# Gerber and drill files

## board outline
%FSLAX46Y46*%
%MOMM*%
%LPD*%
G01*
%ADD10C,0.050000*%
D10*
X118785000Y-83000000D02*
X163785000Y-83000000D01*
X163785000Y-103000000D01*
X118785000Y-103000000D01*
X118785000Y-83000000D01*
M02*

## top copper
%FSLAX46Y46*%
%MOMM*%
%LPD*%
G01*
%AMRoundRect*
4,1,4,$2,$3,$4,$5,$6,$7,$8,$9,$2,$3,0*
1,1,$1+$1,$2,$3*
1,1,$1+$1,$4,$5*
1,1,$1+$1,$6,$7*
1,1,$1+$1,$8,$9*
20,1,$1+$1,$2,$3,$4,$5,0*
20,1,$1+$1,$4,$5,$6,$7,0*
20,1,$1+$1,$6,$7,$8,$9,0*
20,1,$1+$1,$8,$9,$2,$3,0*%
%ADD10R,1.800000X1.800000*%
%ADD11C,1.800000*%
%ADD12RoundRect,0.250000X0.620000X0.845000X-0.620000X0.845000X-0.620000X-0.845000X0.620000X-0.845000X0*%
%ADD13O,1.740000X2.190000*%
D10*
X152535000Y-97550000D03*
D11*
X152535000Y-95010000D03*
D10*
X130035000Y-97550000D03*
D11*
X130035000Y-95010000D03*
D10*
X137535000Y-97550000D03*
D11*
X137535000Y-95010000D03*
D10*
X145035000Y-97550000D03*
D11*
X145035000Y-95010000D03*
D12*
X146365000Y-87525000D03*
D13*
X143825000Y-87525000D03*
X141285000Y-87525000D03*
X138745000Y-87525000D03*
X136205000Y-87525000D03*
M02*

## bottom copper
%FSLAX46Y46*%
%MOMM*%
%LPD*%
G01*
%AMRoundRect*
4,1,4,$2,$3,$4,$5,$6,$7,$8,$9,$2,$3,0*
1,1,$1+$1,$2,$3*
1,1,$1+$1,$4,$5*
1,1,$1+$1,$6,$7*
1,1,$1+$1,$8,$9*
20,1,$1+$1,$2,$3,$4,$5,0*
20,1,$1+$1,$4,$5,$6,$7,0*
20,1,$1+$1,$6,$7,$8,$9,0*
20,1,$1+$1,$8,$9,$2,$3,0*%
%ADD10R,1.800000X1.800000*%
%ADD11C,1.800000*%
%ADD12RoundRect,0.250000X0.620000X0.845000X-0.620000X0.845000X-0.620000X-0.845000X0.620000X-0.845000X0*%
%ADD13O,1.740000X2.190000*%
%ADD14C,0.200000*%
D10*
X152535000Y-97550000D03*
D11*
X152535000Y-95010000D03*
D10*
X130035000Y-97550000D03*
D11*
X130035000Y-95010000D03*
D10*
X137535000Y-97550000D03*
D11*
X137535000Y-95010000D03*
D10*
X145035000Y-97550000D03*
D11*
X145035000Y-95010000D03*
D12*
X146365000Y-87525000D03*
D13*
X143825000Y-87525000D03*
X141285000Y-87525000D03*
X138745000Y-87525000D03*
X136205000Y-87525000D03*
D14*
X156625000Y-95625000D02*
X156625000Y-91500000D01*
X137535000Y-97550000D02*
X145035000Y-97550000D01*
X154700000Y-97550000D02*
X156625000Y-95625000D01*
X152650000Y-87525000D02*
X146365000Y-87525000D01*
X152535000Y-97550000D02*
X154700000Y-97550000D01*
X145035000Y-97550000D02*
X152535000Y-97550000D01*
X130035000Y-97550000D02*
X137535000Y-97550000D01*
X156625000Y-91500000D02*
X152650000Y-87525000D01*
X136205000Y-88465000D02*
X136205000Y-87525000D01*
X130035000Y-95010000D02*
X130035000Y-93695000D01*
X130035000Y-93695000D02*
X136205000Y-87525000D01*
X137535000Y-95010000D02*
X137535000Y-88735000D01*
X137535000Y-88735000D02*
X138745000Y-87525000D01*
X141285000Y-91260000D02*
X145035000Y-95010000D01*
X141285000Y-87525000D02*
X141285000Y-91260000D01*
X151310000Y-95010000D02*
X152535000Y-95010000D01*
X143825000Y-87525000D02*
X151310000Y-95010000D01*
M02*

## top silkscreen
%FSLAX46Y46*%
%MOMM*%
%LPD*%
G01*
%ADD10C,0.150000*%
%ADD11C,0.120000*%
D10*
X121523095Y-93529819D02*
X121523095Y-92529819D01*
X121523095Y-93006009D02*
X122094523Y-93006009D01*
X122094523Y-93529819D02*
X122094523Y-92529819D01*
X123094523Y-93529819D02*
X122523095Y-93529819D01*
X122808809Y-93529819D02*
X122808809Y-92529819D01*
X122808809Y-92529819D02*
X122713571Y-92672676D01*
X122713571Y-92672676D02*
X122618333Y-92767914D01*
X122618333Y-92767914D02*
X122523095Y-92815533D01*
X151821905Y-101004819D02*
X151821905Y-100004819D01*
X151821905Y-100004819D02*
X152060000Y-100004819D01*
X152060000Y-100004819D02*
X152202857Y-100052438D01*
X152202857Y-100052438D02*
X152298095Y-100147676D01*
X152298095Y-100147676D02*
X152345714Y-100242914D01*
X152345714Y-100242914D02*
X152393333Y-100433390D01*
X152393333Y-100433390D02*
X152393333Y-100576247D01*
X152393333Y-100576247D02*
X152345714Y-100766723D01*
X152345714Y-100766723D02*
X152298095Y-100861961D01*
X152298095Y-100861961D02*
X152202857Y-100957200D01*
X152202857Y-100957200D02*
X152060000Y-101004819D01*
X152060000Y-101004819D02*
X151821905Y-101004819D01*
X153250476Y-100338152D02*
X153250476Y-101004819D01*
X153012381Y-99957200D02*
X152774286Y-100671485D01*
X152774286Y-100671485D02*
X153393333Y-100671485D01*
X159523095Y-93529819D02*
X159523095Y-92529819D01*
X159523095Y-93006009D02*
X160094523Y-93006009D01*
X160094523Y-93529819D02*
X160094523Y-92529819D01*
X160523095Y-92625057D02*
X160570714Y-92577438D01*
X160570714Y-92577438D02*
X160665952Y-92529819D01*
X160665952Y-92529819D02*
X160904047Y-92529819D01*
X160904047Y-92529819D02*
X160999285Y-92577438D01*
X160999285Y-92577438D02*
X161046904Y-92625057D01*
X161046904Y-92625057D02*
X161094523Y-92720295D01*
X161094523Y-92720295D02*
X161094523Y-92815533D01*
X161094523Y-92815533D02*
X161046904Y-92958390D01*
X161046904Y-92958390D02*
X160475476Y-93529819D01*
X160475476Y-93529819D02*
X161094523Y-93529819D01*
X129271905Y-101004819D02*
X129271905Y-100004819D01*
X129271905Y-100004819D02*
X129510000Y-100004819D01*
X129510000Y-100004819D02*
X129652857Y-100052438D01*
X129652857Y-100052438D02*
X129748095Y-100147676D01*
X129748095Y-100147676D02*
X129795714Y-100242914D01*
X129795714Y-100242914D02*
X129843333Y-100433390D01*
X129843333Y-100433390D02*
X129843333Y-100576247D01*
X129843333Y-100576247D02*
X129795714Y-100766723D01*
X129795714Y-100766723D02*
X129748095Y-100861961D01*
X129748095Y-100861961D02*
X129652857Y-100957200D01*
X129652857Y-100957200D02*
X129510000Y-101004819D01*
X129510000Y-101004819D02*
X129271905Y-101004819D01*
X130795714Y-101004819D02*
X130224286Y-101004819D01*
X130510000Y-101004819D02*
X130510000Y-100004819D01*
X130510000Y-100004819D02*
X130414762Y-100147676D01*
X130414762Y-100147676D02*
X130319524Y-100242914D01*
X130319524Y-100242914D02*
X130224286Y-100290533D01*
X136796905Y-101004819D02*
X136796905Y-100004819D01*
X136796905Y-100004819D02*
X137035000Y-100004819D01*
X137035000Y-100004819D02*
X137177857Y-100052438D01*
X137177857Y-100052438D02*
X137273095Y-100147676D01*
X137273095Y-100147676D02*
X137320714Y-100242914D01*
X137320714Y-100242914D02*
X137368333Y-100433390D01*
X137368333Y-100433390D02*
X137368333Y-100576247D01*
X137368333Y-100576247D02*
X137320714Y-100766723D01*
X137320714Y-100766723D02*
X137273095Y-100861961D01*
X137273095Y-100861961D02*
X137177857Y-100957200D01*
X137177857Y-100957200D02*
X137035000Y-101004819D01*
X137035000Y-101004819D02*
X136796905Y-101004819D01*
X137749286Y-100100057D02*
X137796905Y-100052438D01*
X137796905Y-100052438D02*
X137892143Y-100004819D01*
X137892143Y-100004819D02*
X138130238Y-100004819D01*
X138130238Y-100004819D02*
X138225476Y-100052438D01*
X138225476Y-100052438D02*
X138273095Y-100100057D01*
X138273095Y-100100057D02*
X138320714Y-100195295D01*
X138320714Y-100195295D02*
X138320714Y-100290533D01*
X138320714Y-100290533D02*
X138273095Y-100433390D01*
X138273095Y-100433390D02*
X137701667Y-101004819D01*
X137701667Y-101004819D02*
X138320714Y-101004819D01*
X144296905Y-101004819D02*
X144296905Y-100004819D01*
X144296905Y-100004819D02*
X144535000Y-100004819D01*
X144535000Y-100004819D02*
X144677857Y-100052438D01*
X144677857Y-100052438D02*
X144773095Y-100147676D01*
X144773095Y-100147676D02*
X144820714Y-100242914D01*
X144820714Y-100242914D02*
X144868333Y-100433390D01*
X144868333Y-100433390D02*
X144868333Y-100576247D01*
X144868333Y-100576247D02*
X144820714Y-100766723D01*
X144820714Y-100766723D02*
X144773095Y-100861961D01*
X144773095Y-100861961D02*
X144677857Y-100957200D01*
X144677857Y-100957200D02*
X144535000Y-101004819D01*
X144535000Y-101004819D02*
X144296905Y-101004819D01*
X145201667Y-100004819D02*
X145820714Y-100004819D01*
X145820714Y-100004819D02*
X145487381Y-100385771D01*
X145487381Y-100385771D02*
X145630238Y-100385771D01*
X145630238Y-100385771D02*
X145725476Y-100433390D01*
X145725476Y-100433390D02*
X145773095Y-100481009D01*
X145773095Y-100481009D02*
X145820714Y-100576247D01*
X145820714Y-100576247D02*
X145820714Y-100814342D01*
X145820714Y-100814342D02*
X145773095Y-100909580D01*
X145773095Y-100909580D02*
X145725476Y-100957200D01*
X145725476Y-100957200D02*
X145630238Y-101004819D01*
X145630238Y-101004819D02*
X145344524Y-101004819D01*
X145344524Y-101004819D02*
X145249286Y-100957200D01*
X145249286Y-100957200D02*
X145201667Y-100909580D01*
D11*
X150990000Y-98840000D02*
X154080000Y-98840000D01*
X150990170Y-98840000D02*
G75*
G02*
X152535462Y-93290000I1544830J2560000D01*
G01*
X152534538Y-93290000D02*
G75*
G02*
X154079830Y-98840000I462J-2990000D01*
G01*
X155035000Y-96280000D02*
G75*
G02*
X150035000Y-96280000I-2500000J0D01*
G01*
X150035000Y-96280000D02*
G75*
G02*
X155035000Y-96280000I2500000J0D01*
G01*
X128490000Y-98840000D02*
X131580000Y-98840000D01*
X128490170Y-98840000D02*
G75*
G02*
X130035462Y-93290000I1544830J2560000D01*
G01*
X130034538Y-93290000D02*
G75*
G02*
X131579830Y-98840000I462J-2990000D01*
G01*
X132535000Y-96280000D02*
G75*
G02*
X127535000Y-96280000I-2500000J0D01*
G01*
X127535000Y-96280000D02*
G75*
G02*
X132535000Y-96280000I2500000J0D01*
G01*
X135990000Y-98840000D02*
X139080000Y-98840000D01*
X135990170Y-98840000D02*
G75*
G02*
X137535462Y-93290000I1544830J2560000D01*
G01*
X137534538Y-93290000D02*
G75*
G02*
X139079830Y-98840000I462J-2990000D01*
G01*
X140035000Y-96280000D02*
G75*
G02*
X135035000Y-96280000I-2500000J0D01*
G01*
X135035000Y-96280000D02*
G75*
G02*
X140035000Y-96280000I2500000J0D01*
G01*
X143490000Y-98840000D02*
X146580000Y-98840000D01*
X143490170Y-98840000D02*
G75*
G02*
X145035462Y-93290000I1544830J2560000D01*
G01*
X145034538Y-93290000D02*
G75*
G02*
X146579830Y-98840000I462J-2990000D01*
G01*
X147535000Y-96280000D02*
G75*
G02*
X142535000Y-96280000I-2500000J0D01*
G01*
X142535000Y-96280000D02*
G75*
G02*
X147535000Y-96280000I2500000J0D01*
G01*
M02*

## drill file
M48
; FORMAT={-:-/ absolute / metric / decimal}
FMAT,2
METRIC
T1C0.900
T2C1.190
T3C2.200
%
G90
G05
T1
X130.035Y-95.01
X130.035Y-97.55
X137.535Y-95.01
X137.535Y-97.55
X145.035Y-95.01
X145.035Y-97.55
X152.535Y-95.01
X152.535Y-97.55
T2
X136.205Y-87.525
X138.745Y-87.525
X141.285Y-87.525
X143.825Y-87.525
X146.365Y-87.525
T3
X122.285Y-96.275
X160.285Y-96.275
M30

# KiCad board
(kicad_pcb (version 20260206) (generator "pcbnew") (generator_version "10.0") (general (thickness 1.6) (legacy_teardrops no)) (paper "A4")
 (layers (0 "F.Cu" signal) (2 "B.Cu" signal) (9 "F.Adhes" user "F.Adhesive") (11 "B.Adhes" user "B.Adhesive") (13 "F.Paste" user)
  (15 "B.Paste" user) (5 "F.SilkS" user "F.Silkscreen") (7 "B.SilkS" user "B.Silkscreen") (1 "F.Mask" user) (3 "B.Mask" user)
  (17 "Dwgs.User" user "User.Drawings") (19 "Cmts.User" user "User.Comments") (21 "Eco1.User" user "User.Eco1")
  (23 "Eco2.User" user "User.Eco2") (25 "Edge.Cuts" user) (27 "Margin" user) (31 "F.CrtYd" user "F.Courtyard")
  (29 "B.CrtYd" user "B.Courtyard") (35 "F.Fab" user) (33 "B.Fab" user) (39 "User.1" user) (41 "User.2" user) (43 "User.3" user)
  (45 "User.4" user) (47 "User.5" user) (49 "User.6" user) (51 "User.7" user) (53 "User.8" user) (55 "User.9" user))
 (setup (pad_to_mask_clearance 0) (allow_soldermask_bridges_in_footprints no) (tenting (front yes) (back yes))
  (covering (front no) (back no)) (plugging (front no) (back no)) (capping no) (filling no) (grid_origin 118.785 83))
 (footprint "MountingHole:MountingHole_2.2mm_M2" (layer "F.Cu") (at 122.285 96.275)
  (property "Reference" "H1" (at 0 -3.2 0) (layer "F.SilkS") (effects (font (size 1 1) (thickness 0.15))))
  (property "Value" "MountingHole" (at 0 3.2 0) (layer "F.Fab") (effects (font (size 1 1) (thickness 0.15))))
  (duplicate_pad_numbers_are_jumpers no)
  (pad "" np_thru_hole circle (at 0 0) (size 2.2 2.2) (drill 2.2) (layers "*.Cu" "*.Mask")))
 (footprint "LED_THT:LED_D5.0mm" (layer "F.Cu") (at 152.535 97.55 90)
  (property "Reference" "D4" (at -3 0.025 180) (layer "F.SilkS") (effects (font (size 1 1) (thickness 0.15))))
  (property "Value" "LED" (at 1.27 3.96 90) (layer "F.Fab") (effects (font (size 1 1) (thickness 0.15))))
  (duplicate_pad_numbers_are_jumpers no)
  (fp_line (start -1.29 -1.545) (end -1.29 1.545) (stroke (width 0.12) (type solid)) (layer "F.SilkS"))
  (fp_arc (start -1.29 -1.54483) (mid 2.072002 -2.880433) (end 4.26 0.000462) (stroke (width 0.12) (type solid)) (layer "F.SilkS"))
  (fp_arc (start 4.26 -0.000462) (mid 2.072002 2.880433) (end -1.29 1.54483) (stroke (width 0.12) (type solid)) (layer "F.SilkS"))
  (fp_circle (center 1.27 0) (end 3.77 0) (stroke (width 0.12) (type solid)) (fill no) (layer "F.SilkS"))
  (pad "1" thru_hole rect (at 0 0 90) (size 1.8 1.8) (drill 0.9) (layers "*.Cu" "*.Mask") (remove_unused_layers no) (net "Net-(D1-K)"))
  (pad "2" thru_hole circle (at 2.54 0 90) (size 1.8 1.8) (drill 0.9) (layers "*.Cu" "*.Mask") (remove_unused_layers no) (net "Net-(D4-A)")))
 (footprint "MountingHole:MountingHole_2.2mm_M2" (layer "F.Cu") (at 160.285 96.275)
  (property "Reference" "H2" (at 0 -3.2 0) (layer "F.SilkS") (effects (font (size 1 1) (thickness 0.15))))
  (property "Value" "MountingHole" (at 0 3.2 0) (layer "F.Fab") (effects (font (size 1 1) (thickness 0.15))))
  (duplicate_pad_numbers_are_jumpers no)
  (pad "" np_thru_hole circle (at 0 0) (size 2.2 2.2) (drill 2.2) (layers "*.Cu" "*.Mask")))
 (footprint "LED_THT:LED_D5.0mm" (layer "F.Cu") (at 130.035 97.55 90)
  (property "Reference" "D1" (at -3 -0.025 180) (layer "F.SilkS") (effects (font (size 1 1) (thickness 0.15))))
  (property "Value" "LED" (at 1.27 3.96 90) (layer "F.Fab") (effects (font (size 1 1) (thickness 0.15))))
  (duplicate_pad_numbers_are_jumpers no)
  (fp_line (start -1.29 -1.545) (end -1.29 1.545) (stroke (width 0.12) (type solid)) (layer "F.SilkS"))
  (fp_arc (start -1.29 -1.54483) (mid 2.072002 -2.880433) (end 4.26 0.000462) (stroke (width 0.12) (type solid)) (layer "F.SilkS"))
  (fp_arc (start 4.26 -0.000462) (mid 2.072002 2.880433) (end -1.29 1.54483) (stroke (width 0.12) (type solid)) (layer "F.SilkS"))
  (fp_circle (center 1.27 0) (end 3.77 0) (stroke (width 0.12) (type solid)) (fill no) (layer "F.SilkS"))
  (pad "1" thru_hole rect (at 0 0 90) (size 1.8 1.8) (drill 0.9) (layers "*.Cu" "*.Mask") (remove_unused_layers no) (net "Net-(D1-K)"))
  (pad "2" thru_hole circle (at 2.54 0 90) (size 1.8 1.8) (drill 0.9) (layers "*.Cu" "*.Mask") (remove_unused_layers no) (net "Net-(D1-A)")))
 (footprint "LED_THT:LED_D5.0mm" (layer "F.Cu") (at 137.535 97.55 90)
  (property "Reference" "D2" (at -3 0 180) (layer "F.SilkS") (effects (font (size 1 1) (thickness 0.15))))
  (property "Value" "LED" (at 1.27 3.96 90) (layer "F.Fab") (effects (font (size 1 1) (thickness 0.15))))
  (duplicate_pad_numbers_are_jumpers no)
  (fp_line (start -1.29 -1.545) (end -1.29 1.545) (stroke (width 0.12) (type solid)) (layer "F.SilkS"))
  (fp_arc (start -1.29 -1.54483) (mid 2.072002 -2.880433) (end 4.26 0.000462) (stroke (width 0.12) (type solid)) (layer "F.SilkS"))
  (fp_arc (start 4.26 -0.000462) (mid 2.072002 2.880433) (end -1.29 1.54483) (stroke (width 0.12) (type solid)) (layer "F.SilkS"))
  (fp_circle (center 1.27 0) (end 3.77 0) (stroke (width 0.12) (type solid)) (fill no) (layer "F.SilkS"))
  (pad "1" thru_hole rect (at 0 0 90) (size 1.8 1.8) (drill 0.9) (layers "*.Cu" "*.Mask") (remove_unused_layers no) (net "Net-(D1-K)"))
  (pad "2" thru_hole circle (at 2.54 0 90) (size 1.8 1.8) (drill 0.9) (layers "*.Cu" "*.Mask") (remove_unused_layers no) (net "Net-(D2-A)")))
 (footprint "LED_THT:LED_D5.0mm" (layer "F.Cu") (at 145.035 97.55 90)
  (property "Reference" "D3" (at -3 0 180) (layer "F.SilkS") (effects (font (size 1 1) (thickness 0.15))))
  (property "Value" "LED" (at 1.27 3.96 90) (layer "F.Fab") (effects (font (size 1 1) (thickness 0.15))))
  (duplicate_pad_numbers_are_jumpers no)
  (fp_line (start -1.29 -1.545) (end -1.29 1.545) (stroke (width 0.12) (type solid)) (layer "F.SilkS"))
  (fp_arc (start -1.29 -1.54483) (mid 2.072002 -2.880433) (end 4.26 0.000462) (stroke (width 0.12) (type solid)) (layer "F.SilkS"))
  (fp_arc (start 4.26 -0.000462) (mid 2.072002 2.880433) (end -1.29 1.54483) (stroke (width 0.12) (type solid)) (layer "F.SilkS"))
  (fp_circle (center 1.27 0) (end 3.77 0) (stroke (width 0.12) (type solid)) (fill no) (layer "F.SilkS"))
  (pad "1" thru_hole rect (at 0 0 90) (size 1.8 1.8) (drill 0.9) (layers "*.Cu" "*.Mask") (remove_unused_layers no) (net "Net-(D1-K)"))
  (pad "2" thru_hole circle (at 2.54 0 90) (size 1.8 1.8) (drill 0.9) (layers "*.Cu" "*.Mask") (remove_unused_layers no) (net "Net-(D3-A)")))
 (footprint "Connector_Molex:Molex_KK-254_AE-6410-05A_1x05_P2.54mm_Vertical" (layer "B.Cu") (at 146.365 87.525 180)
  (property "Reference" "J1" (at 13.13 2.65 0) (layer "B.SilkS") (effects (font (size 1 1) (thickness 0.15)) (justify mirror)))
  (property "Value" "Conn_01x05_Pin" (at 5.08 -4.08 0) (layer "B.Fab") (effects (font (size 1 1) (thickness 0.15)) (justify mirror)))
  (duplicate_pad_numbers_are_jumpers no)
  (pad "1" thru_hole roundrect (at 0 0 180) (size 1.74 2.19) (drill 1.19) (layers "*.Cu" "*.Mask") (remove_unused_layers no)
   (roundrect_rratio 0.1436781609) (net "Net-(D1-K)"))
  (pad "2" thru_hole oval (at 2.54 0 180) (size 1.74 2.19) (drill 1.19) (layers "*.Cu" "*.Mask") (remove_unused_layers no)
   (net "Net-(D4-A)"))
  (pad "3" thru_hole oval (at 5.08 0 180) (size 1.74 2.19) (drill 1.19) (layers "*.Cu" "*.Mask") (remove_unused_layers no)
   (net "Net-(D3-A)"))
  (pad "4" thru_hole oval (at 7.62 0 180) (size 1.74 2.19) (drill 1.19) (layers "*.Cu" "*.Mask") (remove_unused_layers no)
   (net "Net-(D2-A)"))
  (pad "5" thru_hole oval (at 10.16 0 180) (size 1.74 2.19) (drill 1.19) (layers "*.Cu" "*.Mask") (remove_unused_layers no)
   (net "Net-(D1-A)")))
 (gr_rect (start 118.785 83) (end 163.785 103) (stroke (width 0.05) (type default)) (fill no) (layer "Edge.Cuts"))
 (segment (start 156.625 95.625) (end 156.625 91.5) (width 0.2) (layer "B.Cu") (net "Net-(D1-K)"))
 (segment (start 137.535 97.55) (end 145.035 97.55) (width 0.2) (layer "B.Cu") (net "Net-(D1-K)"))
 (segment (start 154.7 97.55) (end 156.625 95.625) (width 0.2) (layer "B.Cu") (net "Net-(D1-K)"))
 (segment (start 152.65 87.525) (end 146.365 87.525) (width 0.2) (layer "B.Cu") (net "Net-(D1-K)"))
 (segment (start 152.535 97.55) (end 154.7 97.55) (width 0.2) (layer "B.Cu") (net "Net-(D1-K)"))
 (segment (start 145.035 97.55) (end 152.535 97.55) (width 0.2) (layer "B.Cu") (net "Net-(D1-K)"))
 (segment (start 130.035 97.55) (end 137.535 97.55) (width 0.2) (layer "B.Cu") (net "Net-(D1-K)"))
 (segment (start 156.625 91.5) (end 152.65 87.525) (width 0.2) (layer "B.Cu") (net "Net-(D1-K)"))
 (segment (start 136.205 88.465) (end 136.205 87.525) (width 0.2) (layer "B.Cu") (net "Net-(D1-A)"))
 (segment (start 130.035 95.01) (end 130.035 93.695) (width 0.2) (layer "B.Cu") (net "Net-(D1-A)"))
 (segment (start 130.035 93.695) (end 136.205 87.525) (width 0.2) (layer "B.Cu") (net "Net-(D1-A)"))
 (segment (start 137.535 95.01) (end 137.535 88.735) (width 0.2) (layer "B.Cu") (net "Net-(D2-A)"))
 (segment (start 137.535 88.735) (end 138.745 87.525) (width 0.2) (layer "B.Cu") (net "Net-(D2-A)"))
 (segment (start 141.285 91.26) (end 145.035 95.01) (width 0.2) (layer "B.Cu") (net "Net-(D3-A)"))
 (segment (start 141.285 87.525) (end 141.285 91.26) (width 0.2) (layer "B.Cu") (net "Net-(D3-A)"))
 (segment (start 151.31 95.01) (end 152.535 95.01) (width 0.2) (layer "B.Cu") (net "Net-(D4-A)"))
 (segment (start 143.825 87.525) (end 151.31 95.01) (width 0.2) (layer "B.Cu") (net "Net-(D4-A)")))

